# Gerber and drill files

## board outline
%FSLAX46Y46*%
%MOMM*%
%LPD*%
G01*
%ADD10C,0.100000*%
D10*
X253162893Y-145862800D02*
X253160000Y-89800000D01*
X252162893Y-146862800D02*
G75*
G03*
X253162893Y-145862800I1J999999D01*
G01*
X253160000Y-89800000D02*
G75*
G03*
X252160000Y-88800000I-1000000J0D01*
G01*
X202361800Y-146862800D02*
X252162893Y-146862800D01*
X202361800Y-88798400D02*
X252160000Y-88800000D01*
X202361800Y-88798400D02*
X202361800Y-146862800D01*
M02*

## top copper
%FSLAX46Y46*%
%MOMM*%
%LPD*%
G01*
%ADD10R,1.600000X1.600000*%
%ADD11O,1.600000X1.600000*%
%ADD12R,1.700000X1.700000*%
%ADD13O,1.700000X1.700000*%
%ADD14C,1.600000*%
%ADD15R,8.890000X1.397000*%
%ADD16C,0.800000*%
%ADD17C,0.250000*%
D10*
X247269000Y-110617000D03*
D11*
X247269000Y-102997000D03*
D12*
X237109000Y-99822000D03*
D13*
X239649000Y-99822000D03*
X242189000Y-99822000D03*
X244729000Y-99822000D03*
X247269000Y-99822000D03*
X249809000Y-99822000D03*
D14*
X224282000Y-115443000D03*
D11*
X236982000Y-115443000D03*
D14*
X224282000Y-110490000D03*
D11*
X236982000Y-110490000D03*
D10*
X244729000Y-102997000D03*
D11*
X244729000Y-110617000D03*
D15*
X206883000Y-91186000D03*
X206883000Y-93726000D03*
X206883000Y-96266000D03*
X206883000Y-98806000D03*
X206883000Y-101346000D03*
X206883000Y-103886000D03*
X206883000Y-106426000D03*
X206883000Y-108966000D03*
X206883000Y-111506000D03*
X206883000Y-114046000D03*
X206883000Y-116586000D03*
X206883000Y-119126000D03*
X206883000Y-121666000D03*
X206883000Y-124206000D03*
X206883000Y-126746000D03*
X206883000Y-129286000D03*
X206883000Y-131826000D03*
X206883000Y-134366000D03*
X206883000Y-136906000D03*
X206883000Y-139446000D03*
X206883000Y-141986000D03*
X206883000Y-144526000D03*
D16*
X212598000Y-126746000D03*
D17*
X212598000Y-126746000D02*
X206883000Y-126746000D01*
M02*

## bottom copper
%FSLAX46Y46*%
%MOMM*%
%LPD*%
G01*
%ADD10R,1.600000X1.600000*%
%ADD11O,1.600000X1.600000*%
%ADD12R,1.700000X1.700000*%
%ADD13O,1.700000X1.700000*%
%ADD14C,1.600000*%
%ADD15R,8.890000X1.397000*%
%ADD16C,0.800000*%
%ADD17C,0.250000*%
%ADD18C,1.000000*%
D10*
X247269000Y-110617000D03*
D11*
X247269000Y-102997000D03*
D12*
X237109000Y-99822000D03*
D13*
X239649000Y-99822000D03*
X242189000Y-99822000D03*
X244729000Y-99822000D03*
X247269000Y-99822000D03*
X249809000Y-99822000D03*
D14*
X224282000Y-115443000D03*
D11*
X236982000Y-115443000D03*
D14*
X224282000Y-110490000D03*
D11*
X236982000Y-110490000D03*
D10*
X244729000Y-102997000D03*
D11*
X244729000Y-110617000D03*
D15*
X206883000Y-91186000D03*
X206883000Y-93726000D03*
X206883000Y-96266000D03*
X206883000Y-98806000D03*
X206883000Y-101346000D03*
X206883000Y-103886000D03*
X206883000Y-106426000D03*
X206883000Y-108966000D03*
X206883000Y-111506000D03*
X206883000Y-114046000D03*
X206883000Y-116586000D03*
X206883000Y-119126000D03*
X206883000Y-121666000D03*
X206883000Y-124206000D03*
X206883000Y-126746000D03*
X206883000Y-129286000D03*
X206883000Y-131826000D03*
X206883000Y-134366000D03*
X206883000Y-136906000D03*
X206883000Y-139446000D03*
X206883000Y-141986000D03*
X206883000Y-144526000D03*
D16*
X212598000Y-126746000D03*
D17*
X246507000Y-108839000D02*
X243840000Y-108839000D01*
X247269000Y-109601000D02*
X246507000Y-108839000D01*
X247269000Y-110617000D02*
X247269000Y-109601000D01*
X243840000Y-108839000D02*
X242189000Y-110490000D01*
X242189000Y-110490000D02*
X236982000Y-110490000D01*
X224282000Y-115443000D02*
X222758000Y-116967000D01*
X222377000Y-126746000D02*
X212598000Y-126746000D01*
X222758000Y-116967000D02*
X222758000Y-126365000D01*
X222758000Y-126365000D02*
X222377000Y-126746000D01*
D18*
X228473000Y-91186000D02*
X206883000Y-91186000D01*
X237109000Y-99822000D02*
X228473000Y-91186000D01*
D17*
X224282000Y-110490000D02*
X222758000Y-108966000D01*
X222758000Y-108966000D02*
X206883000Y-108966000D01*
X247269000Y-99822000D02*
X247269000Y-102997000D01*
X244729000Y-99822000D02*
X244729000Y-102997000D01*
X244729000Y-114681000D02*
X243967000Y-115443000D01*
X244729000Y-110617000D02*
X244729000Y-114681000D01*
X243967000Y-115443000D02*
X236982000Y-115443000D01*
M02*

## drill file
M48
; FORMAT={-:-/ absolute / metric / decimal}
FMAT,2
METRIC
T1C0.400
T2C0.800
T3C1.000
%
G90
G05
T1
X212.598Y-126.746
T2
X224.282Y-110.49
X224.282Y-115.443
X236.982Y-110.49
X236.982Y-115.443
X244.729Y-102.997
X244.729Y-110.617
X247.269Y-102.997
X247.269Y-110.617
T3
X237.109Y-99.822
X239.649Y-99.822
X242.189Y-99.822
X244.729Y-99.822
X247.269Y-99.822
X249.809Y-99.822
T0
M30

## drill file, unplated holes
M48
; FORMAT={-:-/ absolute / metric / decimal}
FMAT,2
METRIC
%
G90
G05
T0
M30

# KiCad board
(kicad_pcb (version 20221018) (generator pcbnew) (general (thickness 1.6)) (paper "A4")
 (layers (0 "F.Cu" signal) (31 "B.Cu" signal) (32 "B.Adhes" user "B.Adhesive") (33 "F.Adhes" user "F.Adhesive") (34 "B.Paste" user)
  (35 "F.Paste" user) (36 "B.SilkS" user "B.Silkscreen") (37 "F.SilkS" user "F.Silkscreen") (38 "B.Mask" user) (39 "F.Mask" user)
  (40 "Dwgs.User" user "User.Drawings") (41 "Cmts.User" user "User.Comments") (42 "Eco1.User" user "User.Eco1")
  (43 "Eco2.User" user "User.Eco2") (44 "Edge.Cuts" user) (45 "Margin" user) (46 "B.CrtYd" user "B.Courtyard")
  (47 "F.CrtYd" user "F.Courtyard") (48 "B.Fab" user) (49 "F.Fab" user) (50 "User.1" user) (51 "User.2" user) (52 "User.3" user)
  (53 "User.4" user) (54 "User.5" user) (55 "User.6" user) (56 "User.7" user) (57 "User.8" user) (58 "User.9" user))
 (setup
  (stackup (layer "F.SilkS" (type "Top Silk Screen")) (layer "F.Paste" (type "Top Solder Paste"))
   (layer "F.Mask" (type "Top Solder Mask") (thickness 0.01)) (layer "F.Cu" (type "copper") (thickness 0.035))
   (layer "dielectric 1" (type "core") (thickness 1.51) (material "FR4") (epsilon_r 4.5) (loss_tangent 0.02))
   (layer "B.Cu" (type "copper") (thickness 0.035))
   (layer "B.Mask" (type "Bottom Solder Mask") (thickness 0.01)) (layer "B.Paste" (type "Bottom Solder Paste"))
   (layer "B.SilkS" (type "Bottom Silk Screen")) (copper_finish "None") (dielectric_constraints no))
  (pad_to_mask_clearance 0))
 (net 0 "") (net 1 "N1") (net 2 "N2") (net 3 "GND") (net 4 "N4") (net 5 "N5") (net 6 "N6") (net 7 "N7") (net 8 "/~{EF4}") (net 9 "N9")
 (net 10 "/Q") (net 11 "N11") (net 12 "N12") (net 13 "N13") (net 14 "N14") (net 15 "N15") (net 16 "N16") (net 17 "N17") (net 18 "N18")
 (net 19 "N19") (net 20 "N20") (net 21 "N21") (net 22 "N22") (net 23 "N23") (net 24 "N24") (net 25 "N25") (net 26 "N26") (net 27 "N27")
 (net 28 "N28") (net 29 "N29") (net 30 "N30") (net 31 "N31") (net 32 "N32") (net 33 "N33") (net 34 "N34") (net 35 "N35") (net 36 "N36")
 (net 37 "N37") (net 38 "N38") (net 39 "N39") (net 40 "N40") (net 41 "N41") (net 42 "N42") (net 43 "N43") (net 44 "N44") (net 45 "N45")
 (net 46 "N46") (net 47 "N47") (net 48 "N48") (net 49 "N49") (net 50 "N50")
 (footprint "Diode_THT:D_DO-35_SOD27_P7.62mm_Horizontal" (layer "F.Cu") (at 247.269 110.617 90)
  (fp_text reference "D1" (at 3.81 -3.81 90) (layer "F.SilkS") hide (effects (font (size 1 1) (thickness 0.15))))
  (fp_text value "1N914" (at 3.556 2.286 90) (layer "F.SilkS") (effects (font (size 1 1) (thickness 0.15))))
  (pad "1" thru_hole rect (at 0 0 90) (size 1.6 1.6) (drill 0.8) (layers "*.Cu" "*.Mask") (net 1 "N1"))
  (pad "2" thru_hole oval (at 7.62 0 90) (size 1.6 1.6) (drill 0.8) (layers "*.Cu" "*.Mask") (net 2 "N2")))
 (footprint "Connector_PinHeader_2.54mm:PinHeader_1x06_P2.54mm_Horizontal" (layer "F.Cu") (at 237.109 99.822 90)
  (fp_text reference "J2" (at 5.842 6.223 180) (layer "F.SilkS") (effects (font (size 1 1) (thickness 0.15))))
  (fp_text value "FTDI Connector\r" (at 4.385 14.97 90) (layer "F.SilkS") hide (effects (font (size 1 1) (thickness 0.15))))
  (pad "1" thru_hole rect (at 0 0 90) (size 1.7 1.7) (drill 1) (layers "*.Cu" "*.Mask") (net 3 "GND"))
  (pad "2" thru_hole oval (at 0 2.54 90) (size 1.7 1.7) (drill 1) (layers "*.Cu" "*.Mask") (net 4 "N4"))
  (pad "3" thru_hole oval (at 0 5.08 90) (size 1.7 1.7) (drill 1) (layers "*.Cu" "*.Mask") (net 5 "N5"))
  (pad "4" thru_hole oval (at 0 7.62 90) (size 1.7 1.7) (drill 1) (layers "*.Cu" "*.Mask") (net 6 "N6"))
  (pad "5" thru_hole oval (at 0 10.16 90) (size 1.7 1.7) (drill 1) (layers "*.Cu" "*.Mask") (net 2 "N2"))
  (pad "6" thru_hole oval (at 0 12.7 90) (size 1.7 1.7) (drill 1) (layers "*.Cu" "*.Mask") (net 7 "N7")))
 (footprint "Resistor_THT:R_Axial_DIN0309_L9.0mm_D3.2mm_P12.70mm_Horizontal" (layer "F.Cu") (at 224.282 115.443)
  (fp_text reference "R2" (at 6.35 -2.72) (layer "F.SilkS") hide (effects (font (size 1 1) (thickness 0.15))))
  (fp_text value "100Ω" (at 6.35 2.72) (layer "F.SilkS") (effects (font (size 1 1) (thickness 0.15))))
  (pad "1" thru_hole circle (at 0 0) (size 1.6 1.6) (drill 0.8) (layers "*.Cu" "*.Mask") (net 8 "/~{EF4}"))
  (pad "2" thru_hole oval (at 12.7 0) (size 1.6 1.6) (drill 0.8) (layers "*.Cu" "*.Mask") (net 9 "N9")))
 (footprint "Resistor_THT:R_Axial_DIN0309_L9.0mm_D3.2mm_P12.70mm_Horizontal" (layer "F.Cu") (at 224.282 110.49)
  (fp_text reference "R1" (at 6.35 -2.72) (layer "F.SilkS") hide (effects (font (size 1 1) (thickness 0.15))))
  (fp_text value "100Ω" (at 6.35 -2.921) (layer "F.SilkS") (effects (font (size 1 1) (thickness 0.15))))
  (pad "1" thru_hole circle (at 0 0) (size 1.6 1.6) (drill 0.8) (layers "*.Cu" "*.Mask") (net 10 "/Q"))
  (pad "2" thru_hole oval (at 12.7 0) (size 1.6 1.6) (drill 0.8) (layers "*.Cu" "*.Mask") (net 1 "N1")))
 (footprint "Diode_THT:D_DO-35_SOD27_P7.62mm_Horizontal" (layer "F.Cu") (at 244.729 102.997 -90)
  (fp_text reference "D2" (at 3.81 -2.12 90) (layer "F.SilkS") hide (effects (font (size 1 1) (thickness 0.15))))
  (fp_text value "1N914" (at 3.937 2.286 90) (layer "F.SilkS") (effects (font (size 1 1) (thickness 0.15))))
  (pad "1" thru_hole rect (at 0 0 270) (size 1.6 1.6) (drill 0.8) (layers "*.Cu" "*.Mask") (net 6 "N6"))
  (pad "2" thru_hole oval (at 7.62 0 270) (size 1.6 1.6) (drill 0.8) (layers "*.Cu" "*.Mask") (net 9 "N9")))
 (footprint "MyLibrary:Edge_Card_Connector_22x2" (layer "F.Cu") (at 206.883 144.526 90)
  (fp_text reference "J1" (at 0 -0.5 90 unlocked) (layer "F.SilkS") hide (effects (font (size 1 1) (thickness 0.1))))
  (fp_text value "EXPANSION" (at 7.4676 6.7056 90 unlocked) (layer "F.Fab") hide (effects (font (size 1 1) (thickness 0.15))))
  (pad "1" connect rect (at 53.34 0 90) (size 1.397 8.89) (layers "B.Cu" "B.Mask") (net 3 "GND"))
  (pad "2" connect rect (at 53.34 0 90) (size 1.397 8.89) (layers "F.Cu" "F.Mask") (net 3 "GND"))
  (pad "3" connect rect (at 50.8 0 90) (size 1.397 8.89) (layers "B.Cu" "B.Mask") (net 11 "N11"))
  (pad "4" connect rect (at 50.8 0 90) (size 1.397 8.89) (layers "F.Cu" "F.Mask") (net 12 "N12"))
  (pad "5" connect rect (at 48.26 0 90) (size 1.397 8.89) (layers "B.Cu" "B.Mask") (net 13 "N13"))
  (pad "6" connect rect (at 48.26 0 90) (size 1.397 8.89) (layers "F.Cu" "F.Mask") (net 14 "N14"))
  (pad "7" connect rect (at 45.72 0 90) (size 1.397 8.89) (layers "B.Cu" "B.Mask") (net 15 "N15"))
  (pad "8" connect rect (at 45.72 0 90) (size 1.397 8.89) (layers "F.Cu" "F.Mask") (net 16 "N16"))
  (pad "9" connect rect (at 43.18 0 90) (size 1.397 8.89) (layers "B.Cu" "B.Mask") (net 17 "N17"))
  (pad "10" connect rect (at 43.18 0 90) (size 1.397 8.89) (layers "F.Cu" "F.Mask") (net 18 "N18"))
  (pad "11" connect rect (at 40.64 0 90) (size 1.397 8.89) (layers "B.Cu" "B.Mask") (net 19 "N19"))
  (pad "12" connect rect (at 40.64 0 90) (size 1.397 8.89) (layers "F.Cu" "F.Mask") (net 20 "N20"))
  (pad "13" connect rect (at 38.1 0 90) (size 1.397 8.89) (layers "B.Cu" "B.Mask") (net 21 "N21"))
  (pad "14" connect rect (at 38.1 0 90) (size 1.397 8.89) (layers "F.Cu" "F.Mask") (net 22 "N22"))
  (pad "15" connect rect (at 35.56 0 90) (size 1.397 8.89) (layers "B.Cu" "B.Mask") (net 10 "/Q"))
  (pad "16" connect rect (at 35.56 0 90) (size 1.397 8.89) (layers "F.Cu" "F.Mask") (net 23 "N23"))
  (pad "17" connect rect (at 33.02 0 90) (size 1.397 8.89) (layers "B.Cu" "B.Mask") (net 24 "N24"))
  (pad "18" connect rect (at 33.02 0 90) (size 1.397 8.89) (layers "F.Cu" "F.Mask") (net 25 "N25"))
  (pad "19" connect rect (at 30.48 0 90) (size 1.397 8.89) (layers "B.Cu" "B.Mask") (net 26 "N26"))
  (pad "20" connect rect (at 30.48 0 90) (size 1.397 8.89) (layers "F.Cu" "F.Mask") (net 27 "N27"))
  (pad "21" connect rect (at 27.94 0 90) (size 1.397 8.89) (layers "B.Cu" "B.Mask") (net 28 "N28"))
  (pad "22" connect rect (at 27.94 0 90) (size 1.397 8.89) (layers "F.Cu" "F.Mask") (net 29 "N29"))
  (pad "23" connect rect (at 25.4 0 90) (size 1.397 8.89) (layers "B.Cu" "B.Mask") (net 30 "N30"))
  (pad "24" connect rect (at 25.4 0 90) (size 1.397 8.89) (layers "F.Cu" "F.Mask") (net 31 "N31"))
  (pad "25" connect rect (at 22.86 0 90) (size 1.397 8.89) (layers "B.Cu" "B.Mask") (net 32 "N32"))
  (pad "26" connect rect (at 22.86 0 90) (size 1.397 8.89) (layers "F.Cu" "F.Mask") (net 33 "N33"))
  (pad "27" connect rect (at 20.32 0 90) (size 1.397 8.89) (layers "B.Cu" "B.Mask") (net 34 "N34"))
  (pad "28" connect rect (at 20.32 0 90) (size 1.397 8.89) (layers "F.Cu" "F.Mask") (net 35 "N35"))
  (pad "29" connect rect (at 17.78 0 90) (size 1.397 8.89) (layers "B.Cu" "B.Mask") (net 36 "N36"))
  (pad "30" connect rect (at 17.78 0 90) (size 1.397 8.89) (layers "F.Cu" "F.Mask") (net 8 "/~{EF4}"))
  (pad "31" connect rect (at 15.24 0 90) (size 1.397 8.89) (layers "B.Cu" "B.Mask") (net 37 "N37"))
  (pad "32" connect rect (at 15.24 0 90) (size 1.397 8.89) (layers "F.Cu" "F.Mask") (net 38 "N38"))
  (pad "33" connect rect (at 12.7 0 90) (size 1.397 8.89) (layers "B.Cu" "B.Mask") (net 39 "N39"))
  (pad "34" connect rect (at 12.7 0 90) (size 1.397 8.89) (layers "F.Cu" "F.Mask") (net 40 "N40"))
  (pad "35" connect rect (at 10.16 0 90) (size 1.397 8.89) (layers "B.Cu" "B.Mask") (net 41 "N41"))
  (pad "36" connect rect (at 10.16 0 90) (size 1.397 8.89) (layers "F.Cu" "F.Mask") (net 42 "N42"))
  (pad "37" connect rect (at 7.62 0 90) (size 1.397 8.89) (layers "B.Cu" "B.Mask") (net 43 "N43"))
  (pad "38" connect rect (at 7.62 0 90) (size 1.397 8.89) (layers "F.Cu" "F.Mask") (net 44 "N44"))
  (pad "39" connect rect (at 5.08 0 90) (size 1.397 8.89) (layers "B.Cu" "B.Mask") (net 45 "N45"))
  (pad "40" connect rect (at 5.08 0 90) (size 1.397 8.89) (layers "F.Cu" "F.Mask") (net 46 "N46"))
  (pad "41" connect rect (at 2.54 0 90) (size 1.397 8.89) (layers "B.Cu" "B.Mask") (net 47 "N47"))
  (pad "42" connect rect (at 2.54 0 90) (size 1.397 8.89) (layers "F.Cu" "F.Mask") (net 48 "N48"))
  (pad "43" connect rect (at 0 0 90) (size 1.397 8.89) (layers "B.Cu" "B.Mask") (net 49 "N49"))
  (pad "44" connect rect (at 0 0 90) (size 1.397 8.89) (layers "F.Cu" "F.Mask") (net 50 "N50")))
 (gr_line (start 253.162893 145.8628) (end 253.16 89.8) (stroke (width 0.1) (type default)) (layer "Edge.Cuts"))
 (gr_line (start 202.3618 146.8628) (end 252.162893 146.8628) (stroke (width 0.1) (type default)) (layer "Edge.Cuts"))
 (gr_arc (start 253.162893 145.8628) (mid 252.87 146.569907) (end 252.162893 146.8628) (stroke (width 0.1) (type default))
  (layer "Edge.Cuts"))
 (gr_arc (start 252.16 88.8) (mid 252.867107 89.092893) (end 253.16 89.8) (stroke (width 0.1) (type default)) (layer "Edge.Cuts"))
 (gr_line (start 202.3618 88.7984) (end 252.16 88.8) (stroke (width 0.1) (type default)) (layer "Edge.Cuts"))
 (gr_line (start 202.3618 88.7984) (end 202.3618 146.8628) (stroke (width 0.1) (type default)) (layer "Edge.Cuts"))
 (segment (start 246.507 108.839) (end 243.84 108.839) (width 0.25) (layer "B.Cu") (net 1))
 (segment (start 247.269 109.601) (end 246.507 108.839) (width 0.25) (layer "B.Cu") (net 1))
 (segment (start 247.269 110.617) (end 247.269 109.601) (width 0.25) (layer "B.Cu") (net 1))
 (segment (start 243.84 108.839) (end 242.189 110.49) (width 0.25) (layer "B.Cu") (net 1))
 (segment (start 242.189 110.49) (end 236.982 110.49) (width 0.25) (layer "B.Cu") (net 1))
 (segment (start 212.598 126.746) (end 206.883 126.746) (width 0.25) (layer "F.Cu") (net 8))
 (via (at 212.598 126.746) (size 0.8) (drill 0.4) (layers "F.Cu" "B.Cu") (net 8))
 (segment (start 224.282 115.443) (end 222.758 116.967) (width 0.25) (layer "B.Cu") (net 8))
 (segment (start 222.377 126.746) (end 212.598 126.746) (width 0.25) (layer "B.Cu") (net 8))
 (segment (start 222.758 116.967) (end 222.758 126.365) (width 0.25) (layer "B.Cu") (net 8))
 (segment (start 222.758 126.365) (end 222.377 126.746) (width 0.25) (layer "B.Cu") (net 8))
 (segment (start 228.473 91.186) (end 206.883 91.186) (width 1) (layer "B.Cu") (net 3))
 (segment (start 237.109 99.822) (end 228.473 91.186) (width 1) (layer "B.Cu") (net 3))
 (segment (start 224.282 110.49) (end 222.758 108.966) (width 0.25) (layer "B.Cu") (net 10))
 (segment (start 222.758 108.966) (end 206.883 108.966) (width 0.25) (layer "B.Cu") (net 10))
 (segment (start 247.269 99.822) (end 247.269 102.997) (width 0.25) (layer "B.Cu") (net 2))
 (segment (start 244.729 99.822) (end 244.729 102.997) (width 0.25) (layer "B.Cu") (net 6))
 (segment (start 244.729 114.681) (end 243.967 115.443) (width 0.25) (layer "B.Cu") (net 9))
 (segment (start 244.729 110.617) (end 244.729 114.681) (width 0.25) (layer "B.Cu") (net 9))
 (segment (start 243.967 115.443) (end 236.982 115.443) (width 0.25) (layer "B.Cu") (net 9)))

